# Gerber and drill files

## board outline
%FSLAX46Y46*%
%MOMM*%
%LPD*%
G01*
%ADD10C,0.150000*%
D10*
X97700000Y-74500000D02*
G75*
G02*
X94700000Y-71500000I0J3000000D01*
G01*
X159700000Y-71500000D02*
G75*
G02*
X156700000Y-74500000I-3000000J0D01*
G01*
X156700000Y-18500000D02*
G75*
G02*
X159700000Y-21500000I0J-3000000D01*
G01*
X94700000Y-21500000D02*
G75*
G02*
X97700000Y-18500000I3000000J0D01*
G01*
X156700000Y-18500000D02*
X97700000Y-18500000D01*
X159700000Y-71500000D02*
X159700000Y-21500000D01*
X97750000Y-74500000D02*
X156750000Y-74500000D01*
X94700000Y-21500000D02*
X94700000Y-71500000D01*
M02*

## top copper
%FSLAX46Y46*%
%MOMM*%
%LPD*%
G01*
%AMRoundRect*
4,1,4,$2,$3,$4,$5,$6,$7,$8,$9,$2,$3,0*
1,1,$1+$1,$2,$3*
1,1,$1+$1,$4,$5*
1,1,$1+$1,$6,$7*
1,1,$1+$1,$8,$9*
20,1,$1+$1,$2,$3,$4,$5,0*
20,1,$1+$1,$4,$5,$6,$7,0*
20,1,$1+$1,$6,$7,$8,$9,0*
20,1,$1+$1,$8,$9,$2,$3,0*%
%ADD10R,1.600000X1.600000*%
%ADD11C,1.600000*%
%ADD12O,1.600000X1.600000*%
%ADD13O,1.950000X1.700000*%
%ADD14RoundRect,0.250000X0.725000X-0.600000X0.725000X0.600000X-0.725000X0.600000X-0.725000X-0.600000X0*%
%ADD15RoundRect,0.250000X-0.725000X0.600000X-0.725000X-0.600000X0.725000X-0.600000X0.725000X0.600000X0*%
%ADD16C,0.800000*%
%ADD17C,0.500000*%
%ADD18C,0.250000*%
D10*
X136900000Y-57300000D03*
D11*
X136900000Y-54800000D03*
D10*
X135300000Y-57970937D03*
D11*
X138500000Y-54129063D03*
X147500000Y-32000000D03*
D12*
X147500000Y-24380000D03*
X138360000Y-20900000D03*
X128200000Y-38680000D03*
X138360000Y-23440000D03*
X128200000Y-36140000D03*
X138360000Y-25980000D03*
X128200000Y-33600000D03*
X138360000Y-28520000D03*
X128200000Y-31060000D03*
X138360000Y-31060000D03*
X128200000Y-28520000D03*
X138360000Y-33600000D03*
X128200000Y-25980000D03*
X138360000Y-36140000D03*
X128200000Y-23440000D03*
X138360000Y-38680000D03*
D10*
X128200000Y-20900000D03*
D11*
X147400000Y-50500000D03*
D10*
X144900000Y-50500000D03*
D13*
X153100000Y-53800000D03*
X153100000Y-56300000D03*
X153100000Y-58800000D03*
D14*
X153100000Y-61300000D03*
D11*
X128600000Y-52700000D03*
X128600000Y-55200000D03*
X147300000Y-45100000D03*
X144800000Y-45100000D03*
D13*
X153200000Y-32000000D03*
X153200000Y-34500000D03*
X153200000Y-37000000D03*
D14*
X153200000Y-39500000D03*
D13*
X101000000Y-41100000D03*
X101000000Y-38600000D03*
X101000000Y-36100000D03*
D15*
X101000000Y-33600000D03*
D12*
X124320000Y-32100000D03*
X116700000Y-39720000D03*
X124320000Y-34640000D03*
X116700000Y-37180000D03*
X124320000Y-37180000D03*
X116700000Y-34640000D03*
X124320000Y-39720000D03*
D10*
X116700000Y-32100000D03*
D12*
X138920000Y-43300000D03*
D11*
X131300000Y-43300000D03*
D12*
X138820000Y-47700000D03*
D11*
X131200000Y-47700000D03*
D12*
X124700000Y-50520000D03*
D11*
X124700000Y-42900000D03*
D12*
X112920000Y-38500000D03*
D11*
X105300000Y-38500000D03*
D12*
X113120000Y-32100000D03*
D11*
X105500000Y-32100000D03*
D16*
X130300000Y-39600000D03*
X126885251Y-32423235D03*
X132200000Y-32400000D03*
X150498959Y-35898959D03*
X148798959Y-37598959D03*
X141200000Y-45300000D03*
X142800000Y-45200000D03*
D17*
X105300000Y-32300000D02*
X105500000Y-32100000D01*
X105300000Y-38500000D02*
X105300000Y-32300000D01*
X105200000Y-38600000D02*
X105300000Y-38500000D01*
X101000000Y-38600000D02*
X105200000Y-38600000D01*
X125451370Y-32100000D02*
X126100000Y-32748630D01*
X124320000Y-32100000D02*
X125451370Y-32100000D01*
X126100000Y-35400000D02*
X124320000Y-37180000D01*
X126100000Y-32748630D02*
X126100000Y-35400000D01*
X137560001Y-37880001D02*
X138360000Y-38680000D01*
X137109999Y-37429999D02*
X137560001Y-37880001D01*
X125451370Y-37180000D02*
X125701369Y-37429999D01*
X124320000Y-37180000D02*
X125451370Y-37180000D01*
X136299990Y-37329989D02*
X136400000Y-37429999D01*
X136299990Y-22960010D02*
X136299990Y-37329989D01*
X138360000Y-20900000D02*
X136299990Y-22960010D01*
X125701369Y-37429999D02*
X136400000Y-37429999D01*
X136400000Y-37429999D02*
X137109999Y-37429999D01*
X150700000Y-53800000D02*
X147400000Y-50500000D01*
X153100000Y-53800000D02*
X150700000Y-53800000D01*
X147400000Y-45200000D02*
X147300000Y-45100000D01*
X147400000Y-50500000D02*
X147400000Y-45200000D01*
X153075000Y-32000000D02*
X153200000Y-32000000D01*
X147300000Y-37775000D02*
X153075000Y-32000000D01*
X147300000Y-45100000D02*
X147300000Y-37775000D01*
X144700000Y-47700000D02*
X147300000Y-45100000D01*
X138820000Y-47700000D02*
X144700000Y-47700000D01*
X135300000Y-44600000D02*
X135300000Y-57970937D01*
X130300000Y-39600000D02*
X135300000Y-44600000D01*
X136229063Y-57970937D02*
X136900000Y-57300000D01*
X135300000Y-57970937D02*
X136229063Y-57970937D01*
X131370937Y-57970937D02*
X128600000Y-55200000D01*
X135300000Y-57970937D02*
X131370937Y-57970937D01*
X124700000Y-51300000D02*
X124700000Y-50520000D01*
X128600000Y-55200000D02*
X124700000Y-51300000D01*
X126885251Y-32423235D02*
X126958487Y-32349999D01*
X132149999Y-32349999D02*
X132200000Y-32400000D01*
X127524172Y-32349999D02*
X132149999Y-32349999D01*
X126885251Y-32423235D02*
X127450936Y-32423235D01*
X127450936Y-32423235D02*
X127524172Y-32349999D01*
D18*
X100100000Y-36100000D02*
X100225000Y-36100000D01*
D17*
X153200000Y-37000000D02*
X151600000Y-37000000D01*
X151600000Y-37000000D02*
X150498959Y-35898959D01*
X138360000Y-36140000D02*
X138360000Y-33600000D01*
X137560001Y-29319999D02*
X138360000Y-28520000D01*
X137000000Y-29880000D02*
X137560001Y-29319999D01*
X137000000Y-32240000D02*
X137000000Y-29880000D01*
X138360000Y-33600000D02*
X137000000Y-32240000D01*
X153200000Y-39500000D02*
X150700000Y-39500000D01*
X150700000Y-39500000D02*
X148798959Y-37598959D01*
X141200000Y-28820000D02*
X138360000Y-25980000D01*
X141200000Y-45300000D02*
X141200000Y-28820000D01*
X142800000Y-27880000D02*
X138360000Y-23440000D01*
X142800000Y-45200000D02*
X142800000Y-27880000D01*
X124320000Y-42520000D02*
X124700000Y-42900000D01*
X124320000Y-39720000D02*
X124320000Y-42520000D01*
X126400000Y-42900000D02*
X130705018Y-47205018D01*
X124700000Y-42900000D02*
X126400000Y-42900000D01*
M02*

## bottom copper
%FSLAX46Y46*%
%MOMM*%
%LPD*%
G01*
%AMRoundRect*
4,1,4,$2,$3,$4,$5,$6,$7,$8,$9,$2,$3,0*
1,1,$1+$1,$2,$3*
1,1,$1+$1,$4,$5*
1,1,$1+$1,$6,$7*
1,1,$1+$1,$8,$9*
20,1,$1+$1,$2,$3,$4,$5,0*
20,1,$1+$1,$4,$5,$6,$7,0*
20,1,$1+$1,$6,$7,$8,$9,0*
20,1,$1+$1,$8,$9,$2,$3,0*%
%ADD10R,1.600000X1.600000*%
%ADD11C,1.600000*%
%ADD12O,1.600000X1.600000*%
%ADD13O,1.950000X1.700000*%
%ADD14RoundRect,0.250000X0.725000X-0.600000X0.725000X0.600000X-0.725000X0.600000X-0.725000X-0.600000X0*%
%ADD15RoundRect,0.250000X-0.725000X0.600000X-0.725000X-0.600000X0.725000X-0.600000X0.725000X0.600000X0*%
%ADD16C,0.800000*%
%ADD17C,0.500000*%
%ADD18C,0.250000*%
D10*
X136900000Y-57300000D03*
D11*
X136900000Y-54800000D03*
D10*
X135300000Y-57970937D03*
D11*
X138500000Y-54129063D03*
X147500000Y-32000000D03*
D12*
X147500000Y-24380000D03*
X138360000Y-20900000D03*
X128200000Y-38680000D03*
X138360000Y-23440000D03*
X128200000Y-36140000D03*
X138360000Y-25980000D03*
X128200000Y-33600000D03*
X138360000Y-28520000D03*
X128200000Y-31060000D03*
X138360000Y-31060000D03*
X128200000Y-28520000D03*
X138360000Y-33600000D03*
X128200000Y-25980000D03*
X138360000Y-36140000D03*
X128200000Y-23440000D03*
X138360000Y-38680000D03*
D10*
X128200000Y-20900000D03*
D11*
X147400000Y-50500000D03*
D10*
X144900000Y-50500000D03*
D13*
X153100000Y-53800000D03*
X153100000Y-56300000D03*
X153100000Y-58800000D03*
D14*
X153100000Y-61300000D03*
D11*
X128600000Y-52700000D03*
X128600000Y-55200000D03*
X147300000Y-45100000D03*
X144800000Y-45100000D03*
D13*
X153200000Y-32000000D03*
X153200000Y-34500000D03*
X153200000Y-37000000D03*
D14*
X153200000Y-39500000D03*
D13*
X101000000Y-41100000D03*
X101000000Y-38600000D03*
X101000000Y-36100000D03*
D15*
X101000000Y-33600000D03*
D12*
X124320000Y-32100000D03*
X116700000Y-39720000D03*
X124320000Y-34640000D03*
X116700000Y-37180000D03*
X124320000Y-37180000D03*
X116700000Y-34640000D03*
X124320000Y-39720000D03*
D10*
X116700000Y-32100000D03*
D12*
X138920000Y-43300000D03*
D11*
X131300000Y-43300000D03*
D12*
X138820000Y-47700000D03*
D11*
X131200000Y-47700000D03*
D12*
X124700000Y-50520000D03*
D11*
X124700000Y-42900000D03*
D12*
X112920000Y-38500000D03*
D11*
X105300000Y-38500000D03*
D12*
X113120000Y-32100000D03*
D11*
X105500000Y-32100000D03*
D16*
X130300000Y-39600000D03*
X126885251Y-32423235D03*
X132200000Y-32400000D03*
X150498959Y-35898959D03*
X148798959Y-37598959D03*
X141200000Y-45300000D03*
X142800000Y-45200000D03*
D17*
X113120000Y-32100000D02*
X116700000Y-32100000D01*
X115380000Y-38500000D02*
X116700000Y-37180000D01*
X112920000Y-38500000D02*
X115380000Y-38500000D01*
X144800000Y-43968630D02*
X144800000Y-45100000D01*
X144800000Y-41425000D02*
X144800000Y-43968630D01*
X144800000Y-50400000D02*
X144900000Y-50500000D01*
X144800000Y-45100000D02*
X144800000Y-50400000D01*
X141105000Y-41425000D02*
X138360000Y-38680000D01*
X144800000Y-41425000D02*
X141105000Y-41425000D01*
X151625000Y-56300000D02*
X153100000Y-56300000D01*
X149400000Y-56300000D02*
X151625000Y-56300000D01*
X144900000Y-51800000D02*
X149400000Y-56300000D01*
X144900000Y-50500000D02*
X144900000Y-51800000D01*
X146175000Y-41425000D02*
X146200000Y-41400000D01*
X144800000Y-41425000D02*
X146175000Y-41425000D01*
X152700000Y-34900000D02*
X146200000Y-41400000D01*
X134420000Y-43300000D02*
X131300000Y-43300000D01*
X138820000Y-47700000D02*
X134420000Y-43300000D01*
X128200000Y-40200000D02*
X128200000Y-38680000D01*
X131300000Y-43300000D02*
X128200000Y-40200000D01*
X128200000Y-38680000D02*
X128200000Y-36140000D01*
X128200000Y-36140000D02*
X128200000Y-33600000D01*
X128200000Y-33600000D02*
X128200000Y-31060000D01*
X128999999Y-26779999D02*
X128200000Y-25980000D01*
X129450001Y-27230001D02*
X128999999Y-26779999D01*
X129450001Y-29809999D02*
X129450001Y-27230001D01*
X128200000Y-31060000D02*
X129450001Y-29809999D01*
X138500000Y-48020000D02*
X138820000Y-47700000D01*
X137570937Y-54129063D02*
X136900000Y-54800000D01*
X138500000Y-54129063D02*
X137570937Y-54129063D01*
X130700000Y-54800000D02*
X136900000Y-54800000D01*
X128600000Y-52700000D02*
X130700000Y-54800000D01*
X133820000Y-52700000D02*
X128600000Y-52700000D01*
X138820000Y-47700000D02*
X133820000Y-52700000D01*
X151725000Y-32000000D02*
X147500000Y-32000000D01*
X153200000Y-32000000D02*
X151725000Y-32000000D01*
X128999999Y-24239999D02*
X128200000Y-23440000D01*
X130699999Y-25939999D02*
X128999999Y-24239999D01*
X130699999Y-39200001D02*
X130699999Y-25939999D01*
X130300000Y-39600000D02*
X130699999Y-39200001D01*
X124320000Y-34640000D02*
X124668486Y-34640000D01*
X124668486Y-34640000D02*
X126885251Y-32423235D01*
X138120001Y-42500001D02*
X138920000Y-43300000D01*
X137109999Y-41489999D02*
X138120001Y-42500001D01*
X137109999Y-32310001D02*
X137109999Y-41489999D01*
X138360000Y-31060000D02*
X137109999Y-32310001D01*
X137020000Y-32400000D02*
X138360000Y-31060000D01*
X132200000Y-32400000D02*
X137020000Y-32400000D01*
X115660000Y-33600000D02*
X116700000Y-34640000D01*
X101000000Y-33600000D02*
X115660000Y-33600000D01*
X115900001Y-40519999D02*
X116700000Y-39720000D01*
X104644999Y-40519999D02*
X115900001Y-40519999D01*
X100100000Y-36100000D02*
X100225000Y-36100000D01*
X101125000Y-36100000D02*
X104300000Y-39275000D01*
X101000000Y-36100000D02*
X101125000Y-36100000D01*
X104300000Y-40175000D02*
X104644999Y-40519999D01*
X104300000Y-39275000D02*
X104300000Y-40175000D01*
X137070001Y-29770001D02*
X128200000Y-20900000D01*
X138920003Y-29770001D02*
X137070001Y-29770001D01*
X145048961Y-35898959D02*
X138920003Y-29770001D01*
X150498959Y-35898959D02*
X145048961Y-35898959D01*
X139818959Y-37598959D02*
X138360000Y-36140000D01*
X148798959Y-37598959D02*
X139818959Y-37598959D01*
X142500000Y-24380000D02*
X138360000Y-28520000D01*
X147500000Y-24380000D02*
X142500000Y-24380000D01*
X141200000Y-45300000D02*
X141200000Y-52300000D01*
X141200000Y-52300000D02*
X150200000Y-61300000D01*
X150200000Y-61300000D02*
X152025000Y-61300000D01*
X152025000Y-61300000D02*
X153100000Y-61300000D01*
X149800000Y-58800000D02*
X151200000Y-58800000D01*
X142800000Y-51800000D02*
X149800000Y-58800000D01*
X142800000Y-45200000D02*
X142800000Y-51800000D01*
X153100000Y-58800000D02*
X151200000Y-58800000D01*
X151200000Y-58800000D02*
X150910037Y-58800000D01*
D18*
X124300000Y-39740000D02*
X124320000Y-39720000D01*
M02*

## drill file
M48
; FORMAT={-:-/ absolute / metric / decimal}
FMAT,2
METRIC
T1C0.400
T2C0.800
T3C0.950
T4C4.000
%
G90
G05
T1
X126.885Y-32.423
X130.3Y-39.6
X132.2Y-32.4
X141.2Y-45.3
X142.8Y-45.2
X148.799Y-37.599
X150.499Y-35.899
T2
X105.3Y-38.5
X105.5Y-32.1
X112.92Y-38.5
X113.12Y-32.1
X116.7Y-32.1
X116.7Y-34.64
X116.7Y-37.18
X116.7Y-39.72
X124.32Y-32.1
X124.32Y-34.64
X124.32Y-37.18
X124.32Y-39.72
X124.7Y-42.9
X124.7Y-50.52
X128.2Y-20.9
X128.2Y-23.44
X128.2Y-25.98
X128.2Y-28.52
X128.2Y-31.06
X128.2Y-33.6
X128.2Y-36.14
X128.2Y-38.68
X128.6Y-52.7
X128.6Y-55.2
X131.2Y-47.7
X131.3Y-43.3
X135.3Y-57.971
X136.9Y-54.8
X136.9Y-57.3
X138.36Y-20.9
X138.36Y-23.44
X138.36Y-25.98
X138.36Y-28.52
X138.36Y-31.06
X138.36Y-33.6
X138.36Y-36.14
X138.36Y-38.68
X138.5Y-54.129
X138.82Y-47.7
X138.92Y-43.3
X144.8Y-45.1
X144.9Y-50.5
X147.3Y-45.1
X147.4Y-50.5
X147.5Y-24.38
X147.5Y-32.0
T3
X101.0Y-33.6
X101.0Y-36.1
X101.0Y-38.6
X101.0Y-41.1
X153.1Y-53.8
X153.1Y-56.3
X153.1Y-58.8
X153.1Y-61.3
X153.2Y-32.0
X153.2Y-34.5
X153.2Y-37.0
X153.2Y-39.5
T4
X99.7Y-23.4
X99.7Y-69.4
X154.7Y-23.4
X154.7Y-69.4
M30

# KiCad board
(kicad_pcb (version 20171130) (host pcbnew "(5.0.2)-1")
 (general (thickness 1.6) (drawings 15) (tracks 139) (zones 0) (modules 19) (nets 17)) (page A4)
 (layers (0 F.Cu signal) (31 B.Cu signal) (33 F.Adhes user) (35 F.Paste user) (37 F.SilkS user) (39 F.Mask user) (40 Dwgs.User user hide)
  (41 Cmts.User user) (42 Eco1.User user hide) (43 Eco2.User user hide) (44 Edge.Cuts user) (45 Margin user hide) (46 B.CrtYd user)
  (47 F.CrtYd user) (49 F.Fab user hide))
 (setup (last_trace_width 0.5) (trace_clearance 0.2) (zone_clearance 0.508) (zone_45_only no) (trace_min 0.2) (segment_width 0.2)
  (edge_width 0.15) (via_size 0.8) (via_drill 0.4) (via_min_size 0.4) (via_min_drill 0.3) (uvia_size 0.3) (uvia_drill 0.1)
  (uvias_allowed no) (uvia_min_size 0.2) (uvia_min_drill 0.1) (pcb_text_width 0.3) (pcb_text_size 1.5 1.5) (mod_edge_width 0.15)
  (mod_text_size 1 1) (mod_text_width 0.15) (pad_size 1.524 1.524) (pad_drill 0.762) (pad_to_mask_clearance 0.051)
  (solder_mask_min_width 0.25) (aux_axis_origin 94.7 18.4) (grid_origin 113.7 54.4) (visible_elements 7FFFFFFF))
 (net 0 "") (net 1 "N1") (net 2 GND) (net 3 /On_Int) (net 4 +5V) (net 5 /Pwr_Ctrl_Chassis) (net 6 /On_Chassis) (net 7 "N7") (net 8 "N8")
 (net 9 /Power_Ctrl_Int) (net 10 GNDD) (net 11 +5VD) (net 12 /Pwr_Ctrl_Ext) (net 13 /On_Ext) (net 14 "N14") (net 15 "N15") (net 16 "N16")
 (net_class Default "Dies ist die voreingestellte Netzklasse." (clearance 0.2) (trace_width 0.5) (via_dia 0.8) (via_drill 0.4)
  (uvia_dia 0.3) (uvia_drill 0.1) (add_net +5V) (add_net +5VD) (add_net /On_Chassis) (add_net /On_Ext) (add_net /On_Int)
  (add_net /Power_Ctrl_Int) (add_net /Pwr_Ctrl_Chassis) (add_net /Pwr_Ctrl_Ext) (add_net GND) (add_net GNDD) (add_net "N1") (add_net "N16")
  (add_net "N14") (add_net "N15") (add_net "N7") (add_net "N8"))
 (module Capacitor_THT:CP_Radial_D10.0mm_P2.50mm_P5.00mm (layer F.Cu) (at 136.9 57.3 90)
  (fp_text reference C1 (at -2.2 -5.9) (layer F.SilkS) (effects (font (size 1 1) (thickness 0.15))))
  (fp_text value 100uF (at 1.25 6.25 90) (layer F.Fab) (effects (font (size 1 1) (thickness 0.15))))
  (pad 1 thru_hole rect (at 0 0 90) (size 1.6 1.6) (drill 0.8) (layers *.Cu *.Mask) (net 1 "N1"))
  (pad 2 thru_hole circle (at 2.5 0 90) (size 1.6 1.6) (drill 0.8) (layers *.Cu *.Mask) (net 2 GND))
  (pad 1 thru_hole rect (at -0.670937 -1.6 90) (size 1.6 1.6) (drill 0.8) (layers *.Cu *.Mask) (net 1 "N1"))
  (pad 2 thru_hole circle (at 3.170937 1.6 90) (size 1.6 1.6) (drill 0.8) (layers *.Cu *.Mask) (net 2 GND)))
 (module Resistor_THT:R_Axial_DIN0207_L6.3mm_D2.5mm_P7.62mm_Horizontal (layer F.Cu) (at 147.5 32 90)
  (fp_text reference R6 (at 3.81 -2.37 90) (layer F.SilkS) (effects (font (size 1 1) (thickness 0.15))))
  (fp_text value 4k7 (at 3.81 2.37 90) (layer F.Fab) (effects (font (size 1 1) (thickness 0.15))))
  (pad 1 thru_hole circle (at 0 0 90) (size 1.6 1.6) (drill 0.8) (layers *.Cu *.Mask) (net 2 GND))
  (pad 2 thru_hole oval (at 7.62 0 90) (size 1.6 1.6) (drill 0.8) (layers *.Cu *.Mask) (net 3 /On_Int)))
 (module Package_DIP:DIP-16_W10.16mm (layer F.Cu) (at 128.2 20.9)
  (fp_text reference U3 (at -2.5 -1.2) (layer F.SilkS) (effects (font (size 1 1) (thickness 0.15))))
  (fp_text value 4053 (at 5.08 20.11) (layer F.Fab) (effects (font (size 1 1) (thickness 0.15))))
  (pad 16 thru_hole oval (at 10.16 0) (size 1.6 1.6) (drill 0.8) (layers *.Cu *.Mask) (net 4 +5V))
  (pad 8 thru_hole oval (at 0 17.78) (size 1.6 1.6) (drill 0.8) (layers *.Cu *.Mask) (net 2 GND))
  (pad 15 thru_hole oval (at 10.16 2.54) (size 1.6 1.6) (drill 0.8) (layers *.Cu *.Mask) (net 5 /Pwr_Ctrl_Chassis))
  (pad 7 thru_hole oval (at 0 15.24) (size 1.6 1.6) (drill 0.8) (layers *.Cu *.Mask) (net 2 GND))
  (pad 14 thru_hole oval (at 10.16 5.08) (size 1.6 1.6) (drill 0.8) (layers *.Cu *.Mask) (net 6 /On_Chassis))
  (pad 6 thru_hole oval (at 0 12.7) (size 1.6 1.6) (drill 0.8) (layers *.Cu *.Mask) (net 2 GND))
  (pad 13 thru_hole oval (at 10.16 7.62) (size 1.6 1.6) (drill 0.8) (layers *.Cu *.Mask) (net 3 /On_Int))
  (pad 5 thru_hole oval (at 0 10.16) (size 1.6 1.6) (drill 0.8) (layers *.Cu *.Mask) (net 2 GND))
  (pad 12 thru_hole oval (at 10.16 10.16) (size 1.6 1.6) (drill 0.8) (layers *.Cu *.Mask) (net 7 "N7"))
  (pad 4 thru_hole oval (at 0 7.62) (size 1.6 1.6) (drill 0.8) (layers *.Cu *.Mask) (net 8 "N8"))
  (pad 11 thru_hole oval (at 10.16 12.7) (size 1.6 1.6) (drill 0.8) (layers *.Cu *.Mask) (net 3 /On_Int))
  (pad 3 thru_hole oval (at 0 5.08) (size 1.6 1.6) (drill 0.8) (layers *.Cu *.Mask) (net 2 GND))
  (pad 10 thru_hole oval (at 10.16 15.24) (size 1.6 1.6) (drill 0.8) (layers *.Cu *.Mask) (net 3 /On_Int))
  (pad 2 thru_hole oval (at 0 2.54) (size 1.6 1.6) (drill 0.8) (layers *.Cu *.Mask) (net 1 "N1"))
  (pad 9 thru_hole oval (at 10.16 17.78) (size 1.6 1.6) (drill 0.8) (layers *.Cu *.Mask) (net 4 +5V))
  (pad 1 thru_hole rect (at 0 0) (size 1.6 1.6) (drill 0.8) (layers *.Cu *.Mask) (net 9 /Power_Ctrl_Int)))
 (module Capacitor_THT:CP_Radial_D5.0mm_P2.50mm (layer F.Cu) (at 144.9 50.5)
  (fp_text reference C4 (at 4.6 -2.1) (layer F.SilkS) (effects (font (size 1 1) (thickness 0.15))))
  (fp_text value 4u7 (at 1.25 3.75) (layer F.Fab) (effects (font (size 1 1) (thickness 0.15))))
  (pad 2 thru_hole circle (at 2.5 0) (size 1.6 1.6) (drill 0.8) (layers *.Cu *.Mask) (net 2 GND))
  (pad 1 thru_hole rect (at 0 0) (size 1.6 1.6) (drill 0.8) (layers *.Cu *.Mask) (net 4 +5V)))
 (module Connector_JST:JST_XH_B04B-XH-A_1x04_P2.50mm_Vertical (layer F.Cu) (at 153.1 61.3 90)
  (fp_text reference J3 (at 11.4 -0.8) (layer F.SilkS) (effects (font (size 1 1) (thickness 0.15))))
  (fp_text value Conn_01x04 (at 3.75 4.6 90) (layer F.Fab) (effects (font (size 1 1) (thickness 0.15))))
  (pad 4 thru_hole oval (at 7.5 0 90) (size 1.7 1.95) (drill 0.95) (layers *.Cu *.Mask) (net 2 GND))
  (pad 3 thru_hole oval (at 5 0 90) (size 1.7 1.95) (drill 0.95) (layers *.Cu *.Mask) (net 4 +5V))
  (pad 2 thru_hole oval (at 2.5 0 90) (size 1.7 1.95) (drill 0.95) (layers *.Cu *.Mask) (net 5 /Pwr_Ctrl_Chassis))
  (pad 1 thru_hole roundrect (at 0 0 90) (size 1.7 1.95) (drill 0.95) (layers *.Cu *.Mask) (roundrect_rratio 0.147059) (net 6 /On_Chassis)))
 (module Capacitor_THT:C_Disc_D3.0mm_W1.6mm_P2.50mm (layer F.Cu) (at 128.6 55.2 90)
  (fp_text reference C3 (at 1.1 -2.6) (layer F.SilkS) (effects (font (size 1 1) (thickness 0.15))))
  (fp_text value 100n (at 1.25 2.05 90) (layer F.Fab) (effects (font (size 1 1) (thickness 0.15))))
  (pad 2 thru_hole circle (at 2.5 0 90) (size 1.6 1.6) (drill 0.8) (layers *.Cu *.Mask) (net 2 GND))
  (pad 1 thru_hole circle (at 0 0 90) (size 1.6 1.6) (drill 0.8) (layers *.Cu *.Mask) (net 1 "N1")))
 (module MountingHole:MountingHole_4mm (layer F.Cu) (at 154.7 69.4)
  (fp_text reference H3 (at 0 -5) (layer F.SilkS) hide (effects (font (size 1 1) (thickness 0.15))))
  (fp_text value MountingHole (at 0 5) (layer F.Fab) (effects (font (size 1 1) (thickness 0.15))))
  (pad 1 np_thru_hole circle (at 0 0) (size 4 4) (drill 4) (layers *.Cu *.Mask)))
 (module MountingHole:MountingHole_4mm (layer F.Cu) (at 154.7 23.4)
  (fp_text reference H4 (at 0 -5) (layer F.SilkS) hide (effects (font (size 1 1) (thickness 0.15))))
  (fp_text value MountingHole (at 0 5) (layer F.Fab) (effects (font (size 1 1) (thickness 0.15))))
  (pad 1 np_thru_hole circle (at 0 0) (size 4 4) (drill 4) (layers *.Cu *.Mask)))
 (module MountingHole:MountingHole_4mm (layer F.Cu) (at 99.7 23.4)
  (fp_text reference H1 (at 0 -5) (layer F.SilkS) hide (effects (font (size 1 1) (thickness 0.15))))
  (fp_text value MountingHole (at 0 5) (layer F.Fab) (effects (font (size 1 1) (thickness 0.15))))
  (pad 1 np_thru_hole circle (at 0 0) (size 4 4) (drill 4) (layers *.Cu *.Mask)))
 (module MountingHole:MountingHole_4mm (layer F.Cu) (at 99.7 69.4)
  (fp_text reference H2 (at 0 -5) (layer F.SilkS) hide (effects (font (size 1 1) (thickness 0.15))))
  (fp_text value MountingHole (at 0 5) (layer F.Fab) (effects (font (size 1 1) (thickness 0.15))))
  (pad 1 np_thru_hole circle (at 0 0) (size 4 4) (drill 4) (layers *.Cu *.Mask)))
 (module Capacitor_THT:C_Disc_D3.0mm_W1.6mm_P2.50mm (layer F.Cu) (at 144.8 45.1)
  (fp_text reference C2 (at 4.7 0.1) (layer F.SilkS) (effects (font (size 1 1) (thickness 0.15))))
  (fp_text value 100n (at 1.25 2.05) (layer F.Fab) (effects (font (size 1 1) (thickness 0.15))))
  (pad 2 thru_hole circle (at 2.5 0) (size 1.6 1.6) (drill 0.8) (layers *.Cu *.Mask) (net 2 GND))
  (pad 1 thru_hole circle (at 0 0) (size 1.6 1.6) (drill 0.8) (layers *.Cu *.Mask) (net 4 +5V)))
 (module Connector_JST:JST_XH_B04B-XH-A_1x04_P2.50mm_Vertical (layer F.Cu) (at 153.2 39.5 90)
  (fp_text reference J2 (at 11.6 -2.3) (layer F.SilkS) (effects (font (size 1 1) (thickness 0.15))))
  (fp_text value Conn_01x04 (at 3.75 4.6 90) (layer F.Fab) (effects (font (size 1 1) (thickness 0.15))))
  (pad 4 thru_hole oval (at 7.5 0 90) (size 1.7 1.95) (drill 0.95) (layers *.Cu *.Mask) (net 2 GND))
  (pad 3 thru_hole oval (at 5 0 90) (size 1.7 1.95) (drill 0.95) (layers *.Cu *.Mask) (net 4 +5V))
  (pad 2 thru_hole oval (at 2.5 0 90) (size 1.7 1.95) (drill 0.95) (layers *.Cu *.Mask) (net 9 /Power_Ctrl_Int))
  (pad 1 thru_hole roundrect (at 0 0 90) (size 1.7 1.95) (drill 0.95) (layers *.Cu *.Mask) (roundrect_rratio 0.147059) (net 3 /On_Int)))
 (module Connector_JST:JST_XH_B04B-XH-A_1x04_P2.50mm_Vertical (layer F.Cu) (at 101 33.6 270)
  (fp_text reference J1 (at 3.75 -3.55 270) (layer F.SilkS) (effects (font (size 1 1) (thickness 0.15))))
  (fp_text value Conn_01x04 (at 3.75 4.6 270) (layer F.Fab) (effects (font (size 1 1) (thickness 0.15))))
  (pad 4 thru_hole oval (at 7.5 0 270) (size 1.7 1.95) (drill 0.95) (layers *.Cu *.Mask) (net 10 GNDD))
  (pad 3 thru_hole oval (at 5 0 270) (size 1.7 1.95) (drill 0.95) (layers *.Cu *.Mask) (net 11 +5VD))
  (pad 2 thru_hole oval (at 2.5 0 270) (size 1.7 1.95) (drill 0.95) (layers *.Cu *.Mask) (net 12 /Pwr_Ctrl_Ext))
  (pad 1 thru_hole roundrect (at 0 0 270) (size 1.7 1.95) (drill 0.95) (layers *.Cu *.Mask) (roundrect_rratio 0.147059) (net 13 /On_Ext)))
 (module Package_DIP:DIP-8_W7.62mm (layer F.Cu) (at 116.7 32.1)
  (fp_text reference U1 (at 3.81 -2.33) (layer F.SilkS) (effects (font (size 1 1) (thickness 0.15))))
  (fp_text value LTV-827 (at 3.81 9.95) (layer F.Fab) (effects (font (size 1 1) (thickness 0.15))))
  (pad 8 thru_hole oval (at 7.62 0) (size 1.6 1.6) (drill 0.8) (layers *.Cu *.Mask) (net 4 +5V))
  (pad 4 thru_hole oval (at 0 7.62) (size 1.6 1.6) (drill 0.8) (layers *.Cu *.Mask) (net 12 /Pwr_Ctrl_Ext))
  (pad 7 thru_hole oval (at 7.62 2.54) (size 1.6 1.6) (drill 0.8) (layers *.Cu *.Mask) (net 7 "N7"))
  (pad 3 thru_hole oval (at 0 5.08) (size 1.6 1.6) (drill 0.8) (layers *.Cu *.Mask) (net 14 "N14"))
  (pad 6 thru_hole oval (at 7.62 5.08) (size 1.6 1.6) (drill 0.8) (layers *.Cu *.Mask) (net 4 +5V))
  (pad 2 thru_hole oval (at 0 2.54) (size 1.6 1.6) (drill 0.8) (layers *.Cu *.Mask) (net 13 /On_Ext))
  (pad 5 thru_hole oval (at 7.62 7.62) (size 1.6 1.6) (drill 0.8) (layers *.Cu *.Mask) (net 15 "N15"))
  (pad 1 thru_hole rect (at 0 0) (size 1.6 1.6) (drill 0.8) (layers *.Cu *.Mask) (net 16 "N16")))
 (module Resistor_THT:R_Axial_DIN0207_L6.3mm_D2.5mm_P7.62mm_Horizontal (layer F.Cu) (at 131.3 43.3)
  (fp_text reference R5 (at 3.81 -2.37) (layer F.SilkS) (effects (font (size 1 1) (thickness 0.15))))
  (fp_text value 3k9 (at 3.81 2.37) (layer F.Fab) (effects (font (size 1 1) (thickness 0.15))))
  (pad 2 thru_hole oval (at 7.62 0) (size 1.6 1.6) (drill 0.8) (layers *.Cu *.Mask) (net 7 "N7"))
  (pad 1 thru_hole circle (at 0 0) (size 1.6 1.6) (drill 0.8) (layers *.Cu *.Mask) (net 2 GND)))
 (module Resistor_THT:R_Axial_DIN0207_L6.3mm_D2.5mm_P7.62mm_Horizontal (layer F.Cu) (at 131.2 47.7)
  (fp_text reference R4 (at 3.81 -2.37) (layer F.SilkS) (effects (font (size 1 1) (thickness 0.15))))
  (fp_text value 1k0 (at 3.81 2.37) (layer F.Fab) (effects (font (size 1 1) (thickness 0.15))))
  (pad 2 thru_hole oval (at 7.62 0) (size 1.6 1.6) (drill 0.8) (layers *.Cu *.Mask) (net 2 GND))
  (pad 1 thru_hole circle (at 0 0) (size 1.6 1.6) (drill 0.8) (layers *.Cu *.Mask) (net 15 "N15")))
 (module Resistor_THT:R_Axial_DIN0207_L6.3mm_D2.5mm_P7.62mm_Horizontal (layer F.Cu) (at 124.7 42.9 270)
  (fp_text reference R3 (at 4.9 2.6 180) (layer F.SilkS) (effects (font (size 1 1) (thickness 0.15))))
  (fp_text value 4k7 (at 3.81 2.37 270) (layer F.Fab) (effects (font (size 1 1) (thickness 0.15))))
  (pad 2 thru_hole oval (at 7.62 0 270) (size 1.6 1.6) (drill 0.8) (layers *.Cu *.Mask) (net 1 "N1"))
  (pad 1 thru_hole circle (at 0 0 270) (size 1.6 1.6) (drill 0.8) (layers *.Cu *.Mask) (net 15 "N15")))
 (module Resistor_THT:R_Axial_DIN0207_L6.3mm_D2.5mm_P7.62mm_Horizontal (layer F.Cu) (at 105.3 38.5)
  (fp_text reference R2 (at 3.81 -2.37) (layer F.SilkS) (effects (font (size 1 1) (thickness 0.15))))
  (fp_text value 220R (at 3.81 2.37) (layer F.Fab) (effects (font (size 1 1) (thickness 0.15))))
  (pad 2 thru_hole oval (at 7.62 0) (size 1.6 1.6) (drill 0.8) (layers *.Cu *.Mask) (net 14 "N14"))
  (pad 1 thru_hole circle (at 0 0) (size 1.6 1.6) (drill 0.8) (layers *.Cu *.Mask) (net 11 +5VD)))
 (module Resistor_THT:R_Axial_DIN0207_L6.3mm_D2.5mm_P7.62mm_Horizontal (layer F.Cu) (at 105.5 32.1)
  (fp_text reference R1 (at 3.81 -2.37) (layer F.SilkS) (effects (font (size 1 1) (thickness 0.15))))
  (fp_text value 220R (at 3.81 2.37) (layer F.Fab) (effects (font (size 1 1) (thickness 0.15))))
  (pad 2 thru_hole oval (at 7.62 0) (size 1.6 1.6) (drill 0.8) (layers *.Cu *.Mask) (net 16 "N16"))
  (pad 1 thru_hole circle (at 0 0) (size 1.6 1.6) (drill 0.8) (layers *.Cu *.Mask) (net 11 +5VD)))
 (gr_arc (start 97.7 71.5) (end 94.7 71.5) (angle -90) (layer Edge.Cuts) (width 0.15))
 (gr_arc (start 156.7 71.5) (end 156.7 74.5) (angle -90) (layer Edge.Cuts) (width 0.15))
 (gr_arc (start 156.7 21.5) (end 159.7 21.5) (angle -90) (layer Edge.Cuts) (width 0.15))
 (gr_arc (start 97.7 21.5) (end 97.7 18.5) (angle -90) (layer Edge.Cuts) (width 0.15))
 (gr_line (start 156.7 18.5) (end 97.7 18.5) (layer Edge.Cuts) (width 0.15))
 (gr_line (start 159.7 71.5) (end 159.7 21.5) (layer Edge.Cuts) (width 0.15))
 (gr_line (start 97.75 74.5) (end 156.75 74.5) (layer Edge.Cuts) (width 0.15))
 (gr_line (start 94.7 21.5) (end 94.7 71.5) (layer Edge.Cuts) (width 0.15))
 (segment (start 105.3 32.3) (end 105.5 32.1) (width 0.5) (layer F.Cu) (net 11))
 (segment (start 105.3 38.5) (end 105.3 32.3) (width 0.5) (layer F.Cu) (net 11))
 (segment (start 105.2 38.6) (end 105.3 38.5) (width 0.5) (layer F.Cu) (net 11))
 (segment (start 101 38.6) (end 105.2 38.6) (width 0.5) (layer F.Cu) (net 11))
 (segment (start 113.12 32.1) (end 116.7 32.1) (width 0.5) (layer B.Cu) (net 16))
 (segment (start 115.38 38.5) (end 116.7 37.18) (width 0.5) (layer B.Cu) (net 14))
 (segment (start 112.92 38.5) (end 115.38 38.5) (width 0.5) (layer B.Cu) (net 14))
 (segment (start 125.45137 32.1) (end 126.1 32.74863) (width 0.5) (layer F.Cu) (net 4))
 (segment (start 124.32 32.1) (end 125.45137 32.1) (width 0.5) (layer F.Cu) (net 4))
 (segment (start 126.1 35.4) (end 124.32 37.18) (width 0.5) (layer F.Cu) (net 4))
 (segment (start 126.1 32.74863) (end 126.1 35.4) (width 0.5) (layer F.Cu) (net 4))
 (segment (start 137.560001 37.880001) (end 138.36 38.68) (width 0.5) (layer F.Cu) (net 4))
 (segment (start 137.109999 37.429999) (end 137.560001 37.880001) (width 0.5) (layer F.Cu) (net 4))
 (segment (start 125.45137 37.18) (end 125.701369 37.429999) (width 0.5) (layer F.Cu) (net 4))
 (segment (start 124.32 37.18) (end 125.45137 37.18) (width 0.5) (layer F.Cu) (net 4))
 (segment (start 136.29999 37.329989) (end 136.4 37.429999) (width 0.5) (layer F.Cu) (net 4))
 (segment (start 136.29999 22.96001) (end 136.29999 37.329989) (width 0.5) (layer F.Cu) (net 4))
 (segment (start 138.36 20.9) (end 136.29999 22.96001) (width 0.5) (layer F.Cu) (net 4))
 (segment (start 125.701369 37.429999) (end 136.4 37.429999) (width 0.5) (layer F.Cu) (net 4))
 (segment (start 136.4 37.429999) (end 137.109999 37.429999) (width 0.5) (layer F.Cu) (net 4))
 (segment (start 144.8 43.96863) (end 144.8 45.1) (width 0.5) (layer B.Cu) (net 4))
 (segment (start 144.8 41.425) (end 144.8 43.96863) (width 0.5) (layer B.Cu) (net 4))
 (segment (start 144.8 50.4) (end 144.9 50.5) (width 0.5) (layer B.Cu) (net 4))
 (segment (start 144.8 45.1) (end 144.8 50.4) (width 0.5) (layer B.Cu) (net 4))
 (segment (start 141.105 41.425) (end 138.36 38.68) (width 0.5) (layer B.Cu) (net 4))
 (segment (start 144.8 41.425) (end 141.105 41.425) (width 0.5) (layer B.Cu) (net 4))
 (segment (start 151.625 56.3) (end 153.1 56.3) (width 0.5) (layer B.Cu) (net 4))
 (segment (start 149.4 56.3) (end 151.625 56.3) (width 0.5) (layer B.Cu) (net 4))
 (segment (start 144.9 51.8) (end 149.4 56.3) (width 0.5) (layer B.Cu) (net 4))
 (segment (start 144.9 50.5) (end 144.9 51.8) (width 0.5) (layer B.Cu) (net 4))
 (segment (start 146.175 41.425) (end 146.2 41.4) (width 0.5) (layer B.Cu) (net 4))
 (segment (start 144.8 41.425) (end 146.175 41.425) (width 0.5) (layer B.Cu) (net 4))
 (segment (start 152.7 34.9) (end 146.2 41.4) (width 0.5) (layer B.Cu) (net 4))
 (segment (start 134.42 43.3) (end 131.3 43.3) (width 0.5) (layer B.Cu) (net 2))
 (segment (start 138.82 47.7) (end 134.42 43.3) (width 0.5) (layer B.Cu) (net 2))
 (segment (start 128.2 40.2) (end 128.2 38.68) (width 0.5) (layer B.Cu) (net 2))
 (segment (start 131.3 43.3) (end 128.2 40.2) (width 0.5) (layer B.Cu) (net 2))
 (segment (start 128.2 38.68) (end 128.2 36.14) (width 0.5) (layer B.Cu) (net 2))
 (segment (start 128.2 36.14) (end 128.2 33.6) (width 0.5) (layer B.Cu) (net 2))
 (segment (start 128.2 33.6) (end 128.2 31.06) (width 0.5) (layer B.Cu) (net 2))
 (segment (start 128.999999 26.779999) (end 128.2 25.98) (width 0.5) (layer B.Cu) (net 2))
 (segment (start 129.450001 27.230001) (end 128.999999 26.779999) (width 0.5) (layer B.Cu) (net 2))
 (segment (start 129.450001 29.809999) (end 129.450001 27.230001) (width 0.5) (layer B.Cu) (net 2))
 (segment (start 128.2 31.06) (end 129.450001 29.809999) (width 0.5) (layer B.Cu) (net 2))
 (segment (start 138.5 48.02) (end 138.82 47.7) (width 0.5) (layer B.Cu) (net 2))
 (segment (start 137.570937 54.129063) (end 136.9 54.8) (width 0.5) (layer B.Cu) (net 2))
 (segment (start 138.5 54.129063) (end 137.570937 54.129063) (width 0.5) (layer B.Cu) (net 2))
 (segment (start 150.7 53.8) (end 147.4 50.5) (width 0.5) (layer F.Cu) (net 2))
 (segment (start 153.1 53.8) (end 150.7 53.8) (width 0.5) (layer F.Cu) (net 2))
 (segment (start 147.4 45.2) (end 147.3 45.1) (width 0.5) (layer F.Cu) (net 2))
 (segment (start 147.4 50.5) (end 147.4 45.2) (width 0.5) (layer F.Cu) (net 2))
 (segment (start 153.075 32) (end 153.2 32) (width 0.5) (layer F.Cu) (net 2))
 (segment (start 147.3 37.775) (end 153.075 32) (width 0.5) (layer F.Cu) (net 2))
 (segment (start 147.3 45.1) (end 147.3 37.775) (width 0.5) (layer F.Cu) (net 2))
 (segment (start 144.7 47.7) (end 147.3 45.1) (width 0.5) (layer F.Cu) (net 2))
 (segment (start 138.82 47.7) (end 144.7 47.7) (width 0.5) (layer F.Cu) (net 2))
 (segment (start 130.7 54.8) (end 136.9 54.8) (width 0.5) (layer B.Cu) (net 2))
 (segment (start 128.6 52.7) (end 130.7 54.8) (width 0.5) (layer B.Cu) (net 2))
 (segment (start 133.82 52.7) (end 128.6 52.7) (width 0.5) (layer B.Cu) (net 2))
 (segment (start 138.82 47.7) (end 133.82 52.7) (width 0.5) (layer B.Cu) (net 2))
 (segment (start 151.725 32) (end 147.5 32) (width 0.5) (layer B.Cu) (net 2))
 (segment (start 153.2 32) (end 151.725 32) (width 0.5) (layer B.Cu) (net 2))
 (via (at 130.3 39.6) (size 0.8) (drill 0.4) (layers F.Cu B.Cu) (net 1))
 (segment (start 128.999999 24.239999) (end 128.2 23.44) (width 0.5) (layer B.Cu) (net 1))
 (segment (start 130.699999 25.939999) (end 128.999999 24.239999) (width 0.5) (layer B.Cu) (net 1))
 (segment (start 130.699999 39.200001) (end 130.699999 25.939999) (width 0.5) (layer B.Cu) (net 1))
 (segment (start 130.3 39.6) (end 130.699999 39.200001) (width 0.5) (layer B.Cu) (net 1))
 (segment (start 135.3 44.6) (end 135.3 57.970937) (width 0.5) (layer F.Cu) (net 1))
 (segment (start 130.3 39.6) (end 135.3 44.6) (width 0.5) (layer F.Cu) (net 1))
 (segment (start 136.229063 57.970937) (end 136.9 57.3) (width 0.5) (layer F.Cu) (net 1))
 (segment (start 135.3 57.970937) (end 136.229063 57.970937) (width 0.5) (layer F.Cu) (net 1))
 (segment (start 131.370937 57.970937) (end 128.6 55.2) (width 0.5) (layer F.Cu) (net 1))
 (segment (start 135.3 57.970937) (end 131.370937 57.970937) (width 0.5) (layer F.Cu) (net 1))
 (segment (start 124.7 51.3) (end 124.7 50.52) (width 0.5) (layer F.Cu) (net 1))
 (segment (start 128.6 55.2) (end 124.7 51.3) (width 0.5) (layer F.Cu) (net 1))
 (via (at 126.885251 32.423235) (size 0.8) (drill 0.4) (layers F.Cu B.Cu) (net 7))
 (segment (start 124.32 34.64) (end 124.668486 34.64) (width 0.5) (layer B.Cu) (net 7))
 (segment (start 124.668486 34.64) (end 126.885251 32.423235) (width 0.5) (layer B.Cu) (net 7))
 (segment (start 126.885251 32.423235) (end 126.958487 32.349999) (width 0.5) (layer F.Cu) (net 7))
 (segment (start 138.120001 42.500001) (end 138.92 43.3) (width 0.5) (layer B.Cu) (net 7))
 (segment (start 137.109999 41.489999) (end 138.120001 42.500001) (width 0.5) (layer B.Cu) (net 7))
 (segment (start 137.109999 32.310001) (end 137.109999 41.489999) (width 0.5) (layer B.Cu) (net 7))
 (segment (start 138.36 31.06) (end 137.109999 32.310001) (width 0.5) (layer B.Cu) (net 7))
 (via (at 132.2 32.4) (size 0.8) (drill 0.4) (layers F.Cu B.Cu) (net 7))
 (segment (start 132.149999 32.349999) (end 132.2 32.4) (width 0.5) (layer F.Cu) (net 7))
 (segment (start 127.524172 32.349999) (end 132.149999 32.349999) (width 0.5) (layer F.Cu) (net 7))
 (segment (start 126.885251 32.423235) (end 127.450936 32.423235) (width 0.5) (layer F.Cu) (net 7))
 (segment (start 127.450936 32.423235) (end 127.524172 32.349999) (width 0.5) (layer F.Cu) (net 7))
 (segment (start 137.02 32.4) (end 138.36 31.06) (width 0.5) (layer B.Cu) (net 7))
 (segment (start 132.2 32.4) (end 137.02 32.4) (width 0.5) (layer B.Cu) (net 7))
 (segment (start 115.66 33.6) (end 116.7 34.64) (width 0.5) (layer B.Cu) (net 13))
 (segment (start 101 33.6) (end 115.66 33.6) (width 0.5) (layer B.Cu) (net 13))
 (segment (start 100.1 36.1) (end 100.225 36.1) (width 0.25) (layer F.Cu) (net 12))
 (segment (start 115.900001 40.519999) (end 116.7 39.72) (width 0.5) (layer B.Cu) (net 12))
 (segment (start 104.644999 40.519999) (end 115.900001 40.519999) (width 0.5) (layer B.Cu) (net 12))
 (segment (start 100.1 36.1) (end 100.225 36.1) (width 0.5) (layer B.Cu) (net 12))
 (segment (start 101.125 36.1) (end 104.3 39.275) (width 0.5) (layer B.Cu) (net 12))
 (segment (start 101 36.1) (end 101.125 36.1) (width 0.5) (layer B.Cu) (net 12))
 (segment (start 104.3 40.175) (end 104.644999 40.519999) (width 0.5) (layer B.Cu) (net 12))
 (segment (start 104.3 39.275) (end 104.3 40.175) (width 0.5) (layer B.Cu) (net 12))
 (via (at 150.498959 35.898959) (size 0.8) (drill 0.4) (layers F.Cu B.Cu) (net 9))
 (segment (start 153.2 37) (end 151.6 37) (width 0.5) (layer F.Cu) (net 9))
 (segment (start 151.6 37) (end 150.498959 35.898959) (width 0.5) (layer F.Cu) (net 9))
 (segment (start 137.070001 29.770001) (end 128.2 20.9) (width 0.5) (layer B.Cu) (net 9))
 (segment (start 138.920003 29.770001) (end 137.070001 29.770001) (width 0.5) (layer B.Cu) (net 9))
 (segment (start 145.048961 35.898959) (end 138.920003 29.770001) (width 0.5) (layer B.Cu) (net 9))
 (segment (start 150.498959 35.898959) (end 145.048961 35.898959) (width 0.5) (layer B.Cu) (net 9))
 (segment (start 138.36 36.14) (end 138.36 33.6) (width 0.5) (layer F.Cu) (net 3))
 (segment (start 137.560001 29.319999) (end 138.36 28.52) (width 0.5) (layer F.Cu) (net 3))
 (segment (start 137 29.88) (end 137.560001 29.319999) (width 0.5) (layer F.Cu) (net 3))
 (segment (start 137 32.24) (end 137 29.88) (width 0.5) (layer F.Cu) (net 3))
 (segment (start 138.36 33.6) (end 137 32.24) (width 0.5) (layer F.Cu) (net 3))
 (via (at 148.798959 37.598959) (size 0.8) (drill 0.4) (layers F.Cu B.Cu) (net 3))
 (segment (start 153.2 39.5) (end 150.7 39.5) (width 0.5) (layer F.Cu) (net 3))
 (segment (start 150.7 39.5) (end 148.798959 37.598959) (width 0.5) (layer F.Cu) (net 3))
 (segment (start 139.818959 37.598959) (end 138.36 36.14) (width 0.5) (layer B.Cu) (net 3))
 (segment (start 148.798959 37.598959) (end 139.818959 37.598959) (width 0.5) (layer B.Cu) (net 3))
 (segment (start 142.5 24.38) (end 138.36 28.52) (width 0.5) (layer B.Cu) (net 3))
 (segment (start 147.5 24.38) (end 142.5 24.38) (width 0.5) (layer B.Cu) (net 3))
 (segment (start 141.2 45.3) (end 141.2 52.3) (width 0.5) (layer B.Cu) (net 6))
 (segment (start 141.2 52.3) (end 150.2 61.3) (width 0.5) (layer B.Cu) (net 6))
 (segment (start 150.2 61.3) (end 152.025 61.3) (width 0.5) (layer B.Cu) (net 6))
 (segment (start 152.025 61.3) (end 153.1 61.3) (width 0.5) (layer B.Cu) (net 6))
 (via (at 141.2 45.3) (size 0.8) (drill 0.4) (layers F.Cu B.Cu) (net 6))
 (segment (start 141.2 28.82) (end 138.36 25.98) (width 0.5) (layer F.Cu) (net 6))
 (segment (start 141.2 45.3) (end 141.2 28.82) (width 0.5) (layer F.Cu) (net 6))
 (via (at 142.8 45.2) (size 0.8) (drill 0.4) (layers F.Cu B.Cu) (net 5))
 (segment (start 149.8 58.8) (end 151.2 58.8) (width 0.5) (layer B.Cu) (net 5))
 (segment (start 142.8 51.8) (end 149.8 58.8) (width 0.5) (layer B.Cu) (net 5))
 (segment (start 142.8 45.2) (end 142.8 51.8) (width 0.5) (layer B.Cu) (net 5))
 (segment (start 153.1 58.8) (end 151.2 58.8) (width 0.5) (layer B.Cu) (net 5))
 (segment (start 151.2 58.8) (end 150.910037 58.8) (width 0.5) (layer B.Cu) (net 5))
 (segment (start 142.8 27.88) (end 138.36 23.44) (width 0.5) (layer F.Cu) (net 5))
 (segment (start 142.8 45.2) (end 142.8 27.88) (width 0.5) (layer F.Cu) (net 5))
 (segment (start 124.3 39.74) (end 124.32 39.72) (width 0.25) (layer B.Cu) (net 15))
 (segment (start 124.32 42.52) (end 124.7 42.9) (width 0.5) (layer F.Cu) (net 15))
 (segment (start 124.32 39.72) (end 124.32 42.52) (width 0.5) (layer F.Cu) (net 15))
 (segment (start 126.4 42.9) (end 130.705018 47.205018) (width 0.5) (layer F.Cu) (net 15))
 (segment (start 124.7 42.9) (end 126.4 42.9) (width 0.5) (layer F.Cu) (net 15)))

